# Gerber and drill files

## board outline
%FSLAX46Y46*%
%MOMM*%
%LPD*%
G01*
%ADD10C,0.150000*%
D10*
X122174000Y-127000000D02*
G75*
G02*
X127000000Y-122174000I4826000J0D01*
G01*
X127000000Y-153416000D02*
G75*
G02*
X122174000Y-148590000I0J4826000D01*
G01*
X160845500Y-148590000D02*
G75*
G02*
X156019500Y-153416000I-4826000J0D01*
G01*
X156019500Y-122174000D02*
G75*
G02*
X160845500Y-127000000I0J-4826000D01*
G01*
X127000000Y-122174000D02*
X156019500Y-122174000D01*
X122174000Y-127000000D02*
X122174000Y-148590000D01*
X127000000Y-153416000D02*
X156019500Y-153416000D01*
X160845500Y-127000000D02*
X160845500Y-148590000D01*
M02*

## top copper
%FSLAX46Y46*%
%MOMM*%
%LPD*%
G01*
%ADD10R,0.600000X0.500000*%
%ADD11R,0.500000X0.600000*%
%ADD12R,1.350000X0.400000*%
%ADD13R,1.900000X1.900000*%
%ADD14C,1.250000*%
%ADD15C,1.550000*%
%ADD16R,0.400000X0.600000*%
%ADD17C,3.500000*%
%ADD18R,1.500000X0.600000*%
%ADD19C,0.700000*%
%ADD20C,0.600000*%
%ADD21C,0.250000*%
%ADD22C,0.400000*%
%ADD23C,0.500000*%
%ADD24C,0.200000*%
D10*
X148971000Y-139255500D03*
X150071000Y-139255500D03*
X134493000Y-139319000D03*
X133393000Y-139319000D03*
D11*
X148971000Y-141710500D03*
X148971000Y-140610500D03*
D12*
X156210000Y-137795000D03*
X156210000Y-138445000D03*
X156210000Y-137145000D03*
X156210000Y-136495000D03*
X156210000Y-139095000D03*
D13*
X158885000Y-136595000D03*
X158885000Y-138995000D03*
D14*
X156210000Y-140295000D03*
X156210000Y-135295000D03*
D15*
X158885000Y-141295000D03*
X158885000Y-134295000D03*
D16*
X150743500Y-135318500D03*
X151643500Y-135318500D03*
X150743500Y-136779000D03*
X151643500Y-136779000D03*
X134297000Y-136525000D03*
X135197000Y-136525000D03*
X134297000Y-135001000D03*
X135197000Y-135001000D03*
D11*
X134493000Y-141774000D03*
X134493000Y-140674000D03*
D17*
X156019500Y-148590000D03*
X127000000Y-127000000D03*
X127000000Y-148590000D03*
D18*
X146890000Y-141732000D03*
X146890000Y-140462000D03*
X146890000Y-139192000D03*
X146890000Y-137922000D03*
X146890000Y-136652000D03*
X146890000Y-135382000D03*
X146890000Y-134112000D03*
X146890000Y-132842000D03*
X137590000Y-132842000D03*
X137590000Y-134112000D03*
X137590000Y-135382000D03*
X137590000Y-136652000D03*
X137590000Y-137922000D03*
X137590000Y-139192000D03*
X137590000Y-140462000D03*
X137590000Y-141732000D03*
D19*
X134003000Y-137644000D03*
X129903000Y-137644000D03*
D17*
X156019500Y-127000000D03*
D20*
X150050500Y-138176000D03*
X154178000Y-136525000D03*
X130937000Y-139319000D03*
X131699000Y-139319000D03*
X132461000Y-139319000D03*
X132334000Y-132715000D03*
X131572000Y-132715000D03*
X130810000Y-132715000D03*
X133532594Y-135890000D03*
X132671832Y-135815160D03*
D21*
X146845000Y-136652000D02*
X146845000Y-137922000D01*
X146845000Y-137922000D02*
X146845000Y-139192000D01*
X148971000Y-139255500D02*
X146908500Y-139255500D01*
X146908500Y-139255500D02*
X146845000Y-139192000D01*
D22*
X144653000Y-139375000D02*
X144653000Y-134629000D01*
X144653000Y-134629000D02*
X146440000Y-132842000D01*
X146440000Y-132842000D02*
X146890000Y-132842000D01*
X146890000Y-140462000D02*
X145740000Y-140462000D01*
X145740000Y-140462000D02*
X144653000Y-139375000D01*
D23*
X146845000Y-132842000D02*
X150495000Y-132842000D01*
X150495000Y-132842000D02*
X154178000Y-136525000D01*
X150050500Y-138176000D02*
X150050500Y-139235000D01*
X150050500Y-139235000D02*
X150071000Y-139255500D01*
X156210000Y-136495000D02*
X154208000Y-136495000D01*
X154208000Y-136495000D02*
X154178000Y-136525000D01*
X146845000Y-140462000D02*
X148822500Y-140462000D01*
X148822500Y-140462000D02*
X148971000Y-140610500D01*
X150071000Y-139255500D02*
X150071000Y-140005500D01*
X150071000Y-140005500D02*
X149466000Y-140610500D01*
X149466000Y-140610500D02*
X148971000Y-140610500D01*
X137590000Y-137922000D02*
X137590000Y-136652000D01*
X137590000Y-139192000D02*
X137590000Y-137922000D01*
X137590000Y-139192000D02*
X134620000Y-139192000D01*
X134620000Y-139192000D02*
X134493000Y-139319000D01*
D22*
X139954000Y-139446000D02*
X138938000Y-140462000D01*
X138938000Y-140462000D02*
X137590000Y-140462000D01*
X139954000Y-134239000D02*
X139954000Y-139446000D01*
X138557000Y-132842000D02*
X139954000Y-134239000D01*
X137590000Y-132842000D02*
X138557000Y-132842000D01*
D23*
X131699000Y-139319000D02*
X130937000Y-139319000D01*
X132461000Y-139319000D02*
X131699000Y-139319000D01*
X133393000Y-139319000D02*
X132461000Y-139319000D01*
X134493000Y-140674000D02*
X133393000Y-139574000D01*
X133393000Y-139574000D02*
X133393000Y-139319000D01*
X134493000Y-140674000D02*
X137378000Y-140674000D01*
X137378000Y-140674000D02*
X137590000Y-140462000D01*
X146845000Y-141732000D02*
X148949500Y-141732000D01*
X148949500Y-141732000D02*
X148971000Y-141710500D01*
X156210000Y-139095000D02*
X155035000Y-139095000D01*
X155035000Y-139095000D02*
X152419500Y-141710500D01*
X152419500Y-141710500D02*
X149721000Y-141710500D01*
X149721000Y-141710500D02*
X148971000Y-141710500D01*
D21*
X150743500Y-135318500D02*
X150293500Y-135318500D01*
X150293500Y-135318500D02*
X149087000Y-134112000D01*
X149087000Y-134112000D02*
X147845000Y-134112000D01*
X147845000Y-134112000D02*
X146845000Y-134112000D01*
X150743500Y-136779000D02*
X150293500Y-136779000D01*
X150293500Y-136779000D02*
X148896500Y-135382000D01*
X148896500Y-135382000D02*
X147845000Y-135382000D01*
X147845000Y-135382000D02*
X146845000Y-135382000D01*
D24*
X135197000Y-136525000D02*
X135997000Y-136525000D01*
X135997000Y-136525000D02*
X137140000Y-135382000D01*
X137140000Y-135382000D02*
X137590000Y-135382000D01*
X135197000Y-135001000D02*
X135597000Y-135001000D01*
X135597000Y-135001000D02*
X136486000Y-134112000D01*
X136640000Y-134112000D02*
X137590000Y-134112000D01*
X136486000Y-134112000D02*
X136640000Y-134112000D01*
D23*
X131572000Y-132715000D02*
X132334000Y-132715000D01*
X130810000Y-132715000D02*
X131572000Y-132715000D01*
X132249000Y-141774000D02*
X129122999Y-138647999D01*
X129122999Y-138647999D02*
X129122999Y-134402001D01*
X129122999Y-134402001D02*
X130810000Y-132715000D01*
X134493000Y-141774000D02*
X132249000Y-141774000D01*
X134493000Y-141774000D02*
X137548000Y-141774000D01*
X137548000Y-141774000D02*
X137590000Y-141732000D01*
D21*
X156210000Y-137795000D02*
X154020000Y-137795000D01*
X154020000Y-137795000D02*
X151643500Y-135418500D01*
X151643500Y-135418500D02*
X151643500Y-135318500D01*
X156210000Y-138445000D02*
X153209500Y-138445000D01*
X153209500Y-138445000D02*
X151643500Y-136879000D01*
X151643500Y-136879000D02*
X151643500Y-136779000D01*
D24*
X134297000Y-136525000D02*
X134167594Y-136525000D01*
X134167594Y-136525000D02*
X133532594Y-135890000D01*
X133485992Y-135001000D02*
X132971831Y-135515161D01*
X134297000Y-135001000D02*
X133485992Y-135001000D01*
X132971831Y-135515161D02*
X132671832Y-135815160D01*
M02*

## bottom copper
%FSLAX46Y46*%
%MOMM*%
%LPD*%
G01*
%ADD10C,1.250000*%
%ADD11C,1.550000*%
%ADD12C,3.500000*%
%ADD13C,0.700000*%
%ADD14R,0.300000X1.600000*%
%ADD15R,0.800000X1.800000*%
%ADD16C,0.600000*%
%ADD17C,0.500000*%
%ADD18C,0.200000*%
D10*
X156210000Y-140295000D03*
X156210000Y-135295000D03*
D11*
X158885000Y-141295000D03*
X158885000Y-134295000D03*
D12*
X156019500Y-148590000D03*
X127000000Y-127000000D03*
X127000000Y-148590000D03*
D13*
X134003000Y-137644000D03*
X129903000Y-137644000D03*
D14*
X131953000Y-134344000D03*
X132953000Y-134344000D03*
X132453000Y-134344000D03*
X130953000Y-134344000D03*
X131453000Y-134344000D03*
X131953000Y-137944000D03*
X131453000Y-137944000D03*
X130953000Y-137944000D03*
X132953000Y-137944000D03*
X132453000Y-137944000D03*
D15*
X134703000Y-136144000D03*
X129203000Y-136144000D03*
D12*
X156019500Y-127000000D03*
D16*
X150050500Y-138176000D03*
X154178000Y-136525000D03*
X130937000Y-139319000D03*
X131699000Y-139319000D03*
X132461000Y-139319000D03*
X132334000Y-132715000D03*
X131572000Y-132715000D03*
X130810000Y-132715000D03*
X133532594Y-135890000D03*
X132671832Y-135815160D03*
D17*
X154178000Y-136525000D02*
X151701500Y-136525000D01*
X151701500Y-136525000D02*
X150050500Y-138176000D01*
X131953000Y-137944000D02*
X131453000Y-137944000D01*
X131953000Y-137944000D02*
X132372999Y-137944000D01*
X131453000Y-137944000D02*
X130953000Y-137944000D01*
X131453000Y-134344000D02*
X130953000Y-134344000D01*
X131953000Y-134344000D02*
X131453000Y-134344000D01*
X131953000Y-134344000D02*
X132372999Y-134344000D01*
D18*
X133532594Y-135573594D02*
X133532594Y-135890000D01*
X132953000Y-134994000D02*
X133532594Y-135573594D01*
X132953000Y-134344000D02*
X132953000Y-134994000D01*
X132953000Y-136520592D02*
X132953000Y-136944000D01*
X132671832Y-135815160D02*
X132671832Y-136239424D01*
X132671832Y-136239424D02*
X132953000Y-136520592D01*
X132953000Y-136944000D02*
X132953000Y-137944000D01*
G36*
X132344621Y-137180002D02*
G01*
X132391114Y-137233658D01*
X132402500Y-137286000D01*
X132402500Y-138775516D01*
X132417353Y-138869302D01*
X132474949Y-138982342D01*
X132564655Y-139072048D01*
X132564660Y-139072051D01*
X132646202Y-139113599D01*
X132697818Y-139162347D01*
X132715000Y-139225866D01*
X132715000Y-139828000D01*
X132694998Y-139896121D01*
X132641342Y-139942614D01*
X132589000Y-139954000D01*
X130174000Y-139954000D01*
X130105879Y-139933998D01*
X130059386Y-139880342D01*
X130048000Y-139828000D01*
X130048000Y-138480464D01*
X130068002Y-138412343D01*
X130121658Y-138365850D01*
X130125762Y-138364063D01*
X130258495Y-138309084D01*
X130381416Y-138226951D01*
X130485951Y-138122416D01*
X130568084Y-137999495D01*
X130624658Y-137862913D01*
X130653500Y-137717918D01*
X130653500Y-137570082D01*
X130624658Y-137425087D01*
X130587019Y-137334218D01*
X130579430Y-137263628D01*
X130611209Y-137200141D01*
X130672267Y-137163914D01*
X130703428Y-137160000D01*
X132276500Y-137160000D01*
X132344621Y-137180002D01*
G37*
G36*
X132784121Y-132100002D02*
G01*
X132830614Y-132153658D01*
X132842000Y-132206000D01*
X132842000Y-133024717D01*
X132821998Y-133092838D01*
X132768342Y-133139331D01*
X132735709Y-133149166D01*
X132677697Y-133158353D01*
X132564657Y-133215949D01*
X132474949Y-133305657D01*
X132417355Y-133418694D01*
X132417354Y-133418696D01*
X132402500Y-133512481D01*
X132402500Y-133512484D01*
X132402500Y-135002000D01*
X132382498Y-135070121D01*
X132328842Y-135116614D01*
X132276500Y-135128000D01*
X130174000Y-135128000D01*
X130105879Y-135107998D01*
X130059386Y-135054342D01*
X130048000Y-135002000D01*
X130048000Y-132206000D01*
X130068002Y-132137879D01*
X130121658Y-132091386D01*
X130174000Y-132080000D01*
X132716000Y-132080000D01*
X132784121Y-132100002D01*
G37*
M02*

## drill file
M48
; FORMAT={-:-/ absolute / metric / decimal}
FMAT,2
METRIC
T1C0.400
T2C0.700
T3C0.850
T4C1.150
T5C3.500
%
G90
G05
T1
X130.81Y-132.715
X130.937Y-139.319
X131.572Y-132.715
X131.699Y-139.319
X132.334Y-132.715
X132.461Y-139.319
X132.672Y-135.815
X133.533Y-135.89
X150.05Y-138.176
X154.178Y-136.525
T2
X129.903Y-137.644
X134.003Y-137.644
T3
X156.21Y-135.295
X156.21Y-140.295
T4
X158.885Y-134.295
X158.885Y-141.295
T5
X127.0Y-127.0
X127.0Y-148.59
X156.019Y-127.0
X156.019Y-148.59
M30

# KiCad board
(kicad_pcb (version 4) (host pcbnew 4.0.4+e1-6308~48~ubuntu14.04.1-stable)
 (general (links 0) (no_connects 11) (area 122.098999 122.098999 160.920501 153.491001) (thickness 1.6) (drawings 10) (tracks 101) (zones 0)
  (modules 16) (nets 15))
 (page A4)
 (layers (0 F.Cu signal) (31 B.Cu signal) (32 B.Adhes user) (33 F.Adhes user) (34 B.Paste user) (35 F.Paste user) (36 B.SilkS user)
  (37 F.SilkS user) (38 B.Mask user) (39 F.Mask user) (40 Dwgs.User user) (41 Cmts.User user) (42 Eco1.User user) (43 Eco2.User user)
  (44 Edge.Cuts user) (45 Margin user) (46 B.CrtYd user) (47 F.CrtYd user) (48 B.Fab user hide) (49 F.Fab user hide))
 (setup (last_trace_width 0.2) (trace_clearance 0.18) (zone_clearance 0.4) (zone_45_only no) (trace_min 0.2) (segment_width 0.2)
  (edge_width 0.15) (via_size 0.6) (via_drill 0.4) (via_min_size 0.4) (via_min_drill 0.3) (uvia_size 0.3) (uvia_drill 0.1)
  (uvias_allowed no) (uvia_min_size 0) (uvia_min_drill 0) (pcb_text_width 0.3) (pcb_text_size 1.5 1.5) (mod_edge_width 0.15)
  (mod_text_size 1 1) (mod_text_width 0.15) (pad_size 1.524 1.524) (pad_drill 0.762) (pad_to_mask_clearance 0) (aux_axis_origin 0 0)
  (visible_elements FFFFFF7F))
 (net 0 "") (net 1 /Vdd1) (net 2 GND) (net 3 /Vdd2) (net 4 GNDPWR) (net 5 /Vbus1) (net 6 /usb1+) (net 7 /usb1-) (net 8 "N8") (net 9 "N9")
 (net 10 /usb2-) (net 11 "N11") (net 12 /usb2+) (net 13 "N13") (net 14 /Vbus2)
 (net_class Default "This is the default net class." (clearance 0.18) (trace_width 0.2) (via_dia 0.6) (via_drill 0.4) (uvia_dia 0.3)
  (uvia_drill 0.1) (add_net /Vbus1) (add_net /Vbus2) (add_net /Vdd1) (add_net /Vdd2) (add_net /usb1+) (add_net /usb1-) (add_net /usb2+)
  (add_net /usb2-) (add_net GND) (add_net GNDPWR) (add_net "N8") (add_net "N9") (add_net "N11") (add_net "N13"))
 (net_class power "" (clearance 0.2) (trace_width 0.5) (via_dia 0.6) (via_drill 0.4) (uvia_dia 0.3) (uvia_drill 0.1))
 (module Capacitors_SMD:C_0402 (layer F.Cu) (at 149.521 139.2555)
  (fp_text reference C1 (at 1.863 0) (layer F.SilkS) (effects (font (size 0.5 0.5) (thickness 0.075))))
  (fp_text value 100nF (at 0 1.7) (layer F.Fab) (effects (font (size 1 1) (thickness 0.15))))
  (pad 1 smd rect (at -0.55 0) (size 0.6 0.5) (layers F.Cu F.Paste F.Mask) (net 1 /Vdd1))
  (pad 2 smd rect (at 0.55 0) (size 0.6 0.5) (layers F.Cu F.Paste F.Mask) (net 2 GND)))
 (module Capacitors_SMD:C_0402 (layer F.Cu) (at 133.943 139.319 180)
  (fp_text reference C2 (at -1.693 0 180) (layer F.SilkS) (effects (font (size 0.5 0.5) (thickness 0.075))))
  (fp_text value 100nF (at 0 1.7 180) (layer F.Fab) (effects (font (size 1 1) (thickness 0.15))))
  (pad 1 smd rect (at -0.55 0 180) (size 0.6 0.5) (layers F.Cu F.Paste F.Mask) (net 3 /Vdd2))
  (pad 2 smd rect (at 0.55 0 180) (size 0.6 0.5) (layers F.Cu F.Paste F.Mask) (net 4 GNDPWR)))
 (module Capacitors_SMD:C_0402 (layer F.Cu) (at 148.971 141.1605 90)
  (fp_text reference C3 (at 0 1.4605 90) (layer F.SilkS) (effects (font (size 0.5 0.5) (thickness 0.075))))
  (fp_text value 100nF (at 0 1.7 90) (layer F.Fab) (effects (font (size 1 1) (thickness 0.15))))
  (pad 1 smd rect (at -0.55 0 90) (size 0.6 0.5) (layers F.Cu F.Paste F.Mask) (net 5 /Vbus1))
  (pad 2 smd rect (at 0.55 0 90) (size 0.6 0.5) (layers F.Cu F.Paste F.Mask) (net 2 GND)))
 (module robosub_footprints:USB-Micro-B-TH (layer F.Cu) (at 155.535 137.795 90)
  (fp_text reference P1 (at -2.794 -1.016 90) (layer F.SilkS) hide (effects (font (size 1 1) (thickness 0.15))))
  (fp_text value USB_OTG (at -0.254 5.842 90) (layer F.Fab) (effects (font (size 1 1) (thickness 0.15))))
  (pad 3 smd rect (at 0 0.675 90) (size 0.4 1.35) (layers F.Cu F.Paste F.Mask) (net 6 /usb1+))
  (pad 2 smd rect (at -0.65 0.675 90) (size 0.4 1.35) (layers F.Cu F.Paste F.Mask) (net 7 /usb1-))
  (pad 4 smd rect (at 0.65 0.675 90) (size 0.4 1.35) (layers F.Cu F.Paste F.Mask))
  (pad 5 smd rect (at 1.3 0.675 90) (size 0.4 1.35) (layers F.Cu F.Paste F.Mask) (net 2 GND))
  (pad 1 smd rect (at -1.3 0.675 90) (size 0.4 1.35) (layers F.Cu F.Paste F.Mask) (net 5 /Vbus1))
  (pad "" smd rect (at 1.2 3.35 90) (size 1.9 1.9) (layers F.Cu F.Paste F.Mask))
  (pad "" smd rect (at -1.2 3.35 90) (size 1.9 1.9) (layers F.Cu F.Paste F.Mask))
  (pad "" thru_hole circle (at -2.5 0.675 90) (size 1.25 1.25) (drill 0.85) (layers *.Cu *.Mask F.SilkS))
  (pad "" thru_hole circle (at 2.5 0.675 90) (size 1.25 1.25) (drill 0.85) (layers *.Cu *.Mask F.SilkS))
  (pad "" thru_hole circle (at -3.5 3.35 90) (size 1.55 1.55) (drill 1.15) (layers *.Cu *.Mask F.SilkS))
  (pad "" thru_hole circle (at 3.5 3.35 90) (size 1.55 1.55) (drill 1.15) (layers *.Cu *.Mask F.SilkS)))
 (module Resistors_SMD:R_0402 (layer F.Cu) (at 151.1935 135.3185)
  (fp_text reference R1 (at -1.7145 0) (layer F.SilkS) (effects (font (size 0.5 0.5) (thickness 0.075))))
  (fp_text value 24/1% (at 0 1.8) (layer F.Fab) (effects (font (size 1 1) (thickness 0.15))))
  (pad 1 smd rect (at -0.45 0) (size 0.4 0.6) (layers F.Cu F.Paste F.Mask) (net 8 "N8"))
  (pad 2 smd rect (at 0.45 0) (size 0.4 0.6) (layers F.Cu F.Paste F.Mask) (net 6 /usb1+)))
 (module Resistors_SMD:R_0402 (layer F.Cu) (at 151.1935 136.779)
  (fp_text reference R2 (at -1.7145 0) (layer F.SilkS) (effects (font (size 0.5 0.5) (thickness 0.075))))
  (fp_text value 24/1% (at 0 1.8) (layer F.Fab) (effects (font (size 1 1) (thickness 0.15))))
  (pad 1 smd rect (at -0.45 0) (size 0.4 0.6) (layers F.Cu F.Paste F.Mask) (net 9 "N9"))
  (pad 2 smd rect (at 0.45 0) (size 0.4 0.6) (layers F.Cu F.Paste F.Mask) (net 7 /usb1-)))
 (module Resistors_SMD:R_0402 (layer F.Cu) (at 134.747 136.525)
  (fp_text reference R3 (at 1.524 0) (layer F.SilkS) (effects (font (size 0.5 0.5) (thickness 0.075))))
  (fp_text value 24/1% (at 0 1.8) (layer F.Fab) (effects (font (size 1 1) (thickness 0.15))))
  (pad 1 smd rect (at -0.45 0) (size 0.4 0.6) (layers F.Cu F.Paste F.Mask) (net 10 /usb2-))
  (pad 2 smd rect (at 0.45 0) (size 0.4 0.6) (layers F.Cu F.Paste F.Mask) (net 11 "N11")))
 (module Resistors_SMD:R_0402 (layer F.Cu) (at 134.747 135.001)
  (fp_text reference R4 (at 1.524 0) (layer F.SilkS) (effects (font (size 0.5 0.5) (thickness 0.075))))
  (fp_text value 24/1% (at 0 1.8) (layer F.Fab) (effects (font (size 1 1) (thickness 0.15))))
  (pad 1 smd rect (at -0.45 0) (size 0.4 0.6) (layers F.Cu F.Paste F.Mask) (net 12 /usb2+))
  (pad 2 smd rect (at 0.45 0) (size 0.4 0.6) (layers F.Cu F.Paste F.Mask) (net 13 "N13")))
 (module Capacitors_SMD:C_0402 (layer F.Cu) (at 134.493 141.224 90)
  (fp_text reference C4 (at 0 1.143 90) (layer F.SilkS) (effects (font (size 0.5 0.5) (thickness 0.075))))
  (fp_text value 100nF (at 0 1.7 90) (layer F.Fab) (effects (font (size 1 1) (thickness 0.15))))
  (pad 1 smd rect (at -0.55 0 90) (size 0.6 0.5) (layers F.Cu F.Paste F.Mask) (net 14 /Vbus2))
  (pad 2 smd rect (at 0.55 0 90) (size 0.6 0.5) (layers F.Cu F.Paste F.Mask) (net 4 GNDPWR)))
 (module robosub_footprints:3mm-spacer (layer F.Cu) (at 156.0195 148.59)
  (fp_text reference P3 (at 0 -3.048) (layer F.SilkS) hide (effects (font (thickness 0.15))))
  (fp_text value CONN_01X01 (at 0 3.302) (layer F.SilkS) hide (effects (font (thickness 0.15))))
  (pad "" thru_hole circle (at 0 0) (size 3.5 3.5) (drill 3.5) (layers *.Cu *.Mask F.SilkS)))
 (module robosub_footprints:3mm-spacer (layer F.Cu) (at 127 127)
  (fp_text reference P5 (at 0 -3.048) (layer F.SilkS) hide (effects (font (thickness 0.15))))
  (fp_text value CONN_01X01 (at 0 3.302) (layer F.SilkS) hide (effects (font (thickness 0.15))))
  (pad "" thru_hole circle (at 0 0) (size 3.5 3.5) (drill 3.5) (layers *.Cu *.Mask F.SilkS)))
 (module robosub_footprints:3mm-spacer (layer F.Cu) (at 127 148.59)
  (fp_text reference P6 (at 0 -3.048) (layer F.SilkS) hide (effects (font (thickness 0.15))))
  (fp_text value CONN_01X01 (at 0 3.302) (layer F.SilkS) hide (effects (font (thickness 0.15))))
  (pad "" thru_hole circle (at 0 0) (size 3.5 3.5) (drill 3.5) (layers *.Cu *.Mask F.SilkS)))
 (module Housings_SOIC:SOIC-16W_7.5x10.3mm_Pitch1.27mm (layer F.Cu) (at 142.24 137.287 180)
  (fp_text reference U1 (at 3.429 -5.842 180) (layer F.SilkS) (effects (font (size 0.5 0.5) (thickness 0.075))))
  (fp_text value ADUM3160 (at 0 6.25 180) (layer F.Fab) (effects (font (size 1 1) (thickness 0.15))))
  (pad 1 smd rect (at -4.65 -4.445 180) (size 1.5 0.6) (layers F.Cu F.Paste F.Mask) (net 5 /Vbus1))
  (pad 2 smd rect (at -4.65 -3.175 180) (size 1.5 0.6) (layers F.Cu F.Paste F.Mask) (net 2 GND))
  (pad 3 smd rect (at -4.65 -1.905 180) (size 1.5 0.6) (layers F.Cu F.Paste F.Mask) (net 1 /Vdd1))
  (pad 4 smd rect (at -4.65 -0.635 180) (size 1.5 0.6) (layers F.Cu F.Paste F.Mask) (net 1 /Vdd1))
  (pad 5 smd rect (at -4.65 0.635 180) (size 1.5 0.6) (layers F.Cu F.Paste F.Mask) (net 1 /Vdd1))
  (pad 6 smd rect (at -4.65 1.905 180) (size 1.5 0.6) (layers F.Cu F.Paste F.Mask) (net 9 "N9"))
  (pad 7 smd rect (at -4.65 3.175 180) (size 1.5 0.6) (layers F.Cu F.Paste F.Mask) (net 8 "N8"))
  (pad 8 smd rect (at -4.65 4.445 180) (size 1.5 0.6) (layers F.Cu F.Paste F.Mask) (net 2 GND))
  (pad 9 smd rect (at 4.65 4.445 180) (size 1.5 0.6) (layers F.Cu F.Paste F.Mask) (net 4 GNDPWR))
  (pad 10 smd rect (at 4.65 3.175 180) (size 1.5 0.6) (layers F.Cu F.Paste F.Mask) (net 13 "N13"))
  (pad 11 smd rect (at 4.65 1.905 180) (size 1.5 0.6) (layers F.Cu F.Paste F.Mask) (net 11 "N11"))
  (pad 12 smd rect (at 4.65 0.635 180) (size 1.5 0.6) (layers F.Cu F.Paste F.Mask) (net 3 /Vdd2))
  (pad 13 smd rect (at 4.65 -0.635 180) (size 1.5 0.6) (layers F.Cu F.Paste F.Mask) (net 3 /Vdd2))
  (pad 14 smd rect (at 4.65 -1.905 180) (size 1.5 0.6) (layers F.Cu F.Paste F.Mask) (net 3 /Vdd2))
  (pad 15 smd rect (at 4.65 -3.175 180) (size 1.5 0.6) (layers F.Cu F.Paste F.Mask) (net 4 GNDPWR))
  (pad 16 smd rect (at 4.65 -4.445 180) (size 1.5 0.6) (layers F.Cu F.Paste F.Mask) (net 14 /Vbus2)))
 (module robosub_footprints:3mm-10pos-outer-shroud (layer B.Cu) (at 131.953 136.144)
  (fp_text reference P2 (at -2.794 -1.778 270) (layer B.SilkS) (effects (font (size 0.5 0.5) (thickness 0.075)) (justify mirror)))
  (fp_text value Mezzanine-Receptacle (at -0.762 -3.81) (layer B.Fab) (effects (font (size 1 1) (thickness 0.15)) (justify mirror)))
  (pad "" thru_hole circle (at 2.05 1.5) (size 0.7 0.7) (drill 0.7) (layers *.Cu *.Mask))
  (pad "" thru_hole circle (at -2.05 1.5) (size 0.7 0.7) (drill 0.7) (layers *.Cu *.Mask))
  (pad 5 smd rect (at 0 -1.8) (size 0.3 1.6) (layers B.Cu B.Paste B.Mask) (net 14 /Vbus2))
  (pad 9 smd rect (at 1 -1.8) (size 0.3 1.6) (layers B.Cu B.Paste B.Mask) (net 10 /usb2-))
  (pad 7 smd rect (at 0.5 -1.8) (size 0.3 1.6) (layers B.Cu B.Paste B.Mask) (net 14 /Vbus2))
  (pad 1 smd rect (at -1 -1.8) (size 0.3 1.6) (layers B.Cu B.Paste B.Mask) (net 14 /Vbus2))
  (pad 3 smd rect (at -0.5 -1.8) (size 0.3 1.6) (layers B.Cu B.Paste B.Mask) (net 14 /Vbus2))
  (pad 6 smd rect (at 0 1.8) (size 0.3 1.6) (layers B.Cu B.Paste B.Mask) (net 4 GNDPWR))
  (pad 4 smd rect (at -0.5 1.8) (size 0.3 1.6) (layers B.Cu B.Paste B.Mask) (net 4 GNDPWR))
  (pad 2 smd rect (at -1 1.8) (size 0.3 1.6) (layers B.Cu B.Paste B.Mask) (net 4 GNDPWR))
  (pad 10 smd rect (at 1 1.8) (size 0.3 1.6) (layers B.Cu B.Paste B.Mask) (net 12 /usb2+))
  (pad 8 smd rect (at 0.5 1.8) (size 0.3 1.6) (layers B.Cu B.Paste B.Mask) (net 4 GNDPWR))
  (pad "" smd rect (at 2.75 0) (size 0.8 1.8) (layers B.Cu B.Paste B.Mask))
  (pad "" smd rect (at -2.75 0) (size 0.8 1.8) (layers B.Cu B.Paste B.Mask)))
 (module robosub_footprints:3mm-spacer (layer F.Cu) (at 156.0195 127)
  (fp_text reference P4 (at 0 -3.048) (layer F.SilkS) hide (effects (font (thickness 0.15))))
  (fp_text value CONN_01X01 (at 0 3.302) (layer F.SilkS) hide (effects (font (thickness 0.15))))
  (pad "" thru_hole circle (at 0 0) (size 3.5 3.5) (drill 3.5) (layers *.Cu *.Mask F.SilkS)))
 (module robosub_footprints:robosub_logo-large (layer F.Cu) (at 141.732 148.717)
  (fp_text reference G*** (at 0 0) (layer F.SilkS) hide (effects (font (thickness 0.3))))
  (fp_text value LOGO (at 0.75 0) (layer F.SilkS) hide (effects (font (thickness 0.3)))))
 (gr_arc (start 127 127) (end 122.174 127) (angle 90) (layer Edge.Cuts) (width 0.15))
 (gr_arc (start 127 148.59) (end 127 153.416) (angle 90) (layer Edge.Cuts) (width 0.15))
 (gr_arc (start 156.0195 148.59) (end 160.8455 148.59) (angle 90) (layer Edge.Cuts) (width 0.15))
 (gr_arc (start 156.0195 127) (end 156.0195 122.174) (angle 90) (layer Edge.Cuts) (width 0.15))
 (gr_line (start 127 122.174) (end 156.0195 122.174) (layer Edge.Cuts) (width 0.15))
 (gr_line (start 122.174 127) (end 122.174 148.59) (layer Edge.Cuts) (width 0.15))
 (gr_line (start 127 153.416) (end 156.0195 153.416) (layer Edge.Cuts) (width 0.15))
 (gr_line (start 160.8455 127) (end 160.8455 148.59) (layer Edge.Cuts) (width 0.15))
 (segment (start 146.845 136.652) (end 146.845 137.922) (width 0.25) (layer F.Cu) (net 1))
 (segment (start 146.845 137.922) (end 146.845 139.192) (width 0.25) (layer F.Cu) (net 1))
 (segment (start 148.971 139.2555) (end 146.9085 139.2555) (width 0.25) (layer F.Cu) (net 1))
 (segment (start 146.9085 139.2555) (end 146.845 139.192) (width 0.25) (layer F.Cu) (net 1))
 (segment (start 144.653 139.375) (end 144.653 134.629) (width 0.4) (layer F.Cu) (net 2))
 (segment (start 144.653 134.629) (end 146.44 132.842) (width 0.4) (layer F.Cu) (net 2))
 (segment (start 146.44 132.842) (end 146.89 132.842) (width 0.4) (layer F.Cu) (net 2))
 (segment (start 146.89 140.462) (end 145.74 140.462) (width 0.4) (layer F.Cu) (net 2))
 (segment (start 145.74 140.462) (end 144.653 139.375) (width 0.4) (layer F.Cu) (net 2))
 (segment (start 146.845 132.842) (end 150.495 132.842) (width 0.5) (layer F.Cu) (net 2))
 (segment (start 150.495 132.842) (end 154.178 136.525) (width 0.5) (layer F.Cu) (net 2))
 (segment (start 150.0505 138.176) (end 150.0505 139.235) (width 0.5) (layer F.Cu) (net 2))
 (segment (start 150.0505 139.235) (end 150.071 139.2555) (width 0.5) (layer F.Cu) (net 2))
 (segment (start 154.178 136.525) (end 151.7015 136.525) (width 0.5) (layer B.Cu) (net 2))
 (segment (start 151.7015 136.525) (end 150.0505 138.176) (width 0.5) (layer B.Cu) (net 2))
 (via (at 150.0505 138.176) (size 0.6) (drill 0.4) (layers F.Cu B.Cu) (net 2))
 (segment (start 156.21 136.495) (end 154.208 136.495) (width 0.5) (layer F.Cu) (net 2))
 (segment (start 154.208 136.495) (end 154.178 136.525) (width 0.5) (layer F.Cu) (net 2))
 (via (at 154.178 136.525) (size 0.6) (drill 0.4) (layers F.Cu B.Cu) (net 2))
 (segment (start 146.845 140.462) (end 148.8225 140.462) (width 0.5) (layer F.Cu) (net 2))
 (segment (start 148.8225 140.462) (end 148.971 140.6105) (width 0.5) (layer F.Cu) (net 2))
 (segment (start 150.071 139.2555) (end 150.071 140.0055) (width 0.5) (layer F.Cu) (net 2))
 (segment (start 150.071 140.0055) (end 149.466 140.6105) (width 0.5) (layer F.Cu) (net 2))
 (segment (start 149.466 140.6105) (end 148.971 140.6105) (width 0.5) (layer F.Cu) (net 2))
 (segment (start 137.59 137.922) (end 137.59 136.652) (width 0.5) (layer F.Cu) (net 3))
 (segment (start 137.59 139.192) (end 137.59 137.922) (width 0.5) (layer F.Cu) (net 3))
 (segment (start 137.59 139.192) (end 134.62 139.192) (width 0.5) (layer F.Cu) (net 3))
 (segment (start 134.62 139.192) (end 134.493 139.319) (width 0.5) (layer F.Cu) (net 3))
 (segment (start 139.954 139.446) (end 138.938 140.462) (width 0.4) (layer F.Cu) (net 4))
 (segment (start 138.938 140.462) (end 137.59 140.462) (width 0.4) (layer F.Cu) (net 4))
 (segment (start 139.954 134.239) (end 139.954 139.446) (width 0.4) (layer F.Cu) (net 4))
 (segment (start 138.557 132.842) (end 139.954 134.239) (width 0.4) (layer F.Cu) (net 4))
 (segment (start 137.59 132.842) (end 138.557 132.842) (width 0.4) (layer F.Cu) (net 4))
 (segment (start 131.953 137.944) (end 131.453 137.944) (width 0.5) (layer B.Cu) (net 4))
 (segment (start 131.699 139.319) (end 130.937 139.319) (width 0.5) (layer F.Cu) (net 4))
 (via (at 130.937 139.319) (size 0.6) (drill 0.4) (layers F.Cu B.Cu) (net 4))
 (segment (start 132.461 139.319) (end 131.699 139.319) (width 0.5) (layer F.Cu) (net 4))
 (via (at 131.699 139.319) (size 0.6) (drill 0.4) (layers F.Cu B.Cu) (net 4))
 (segment (start 133.393 139.319) (end 132.461 139.319) (width 0.5) (layer F.Cu) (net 4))
 (via (at 132.461 139.319) (size 0.6) (drill 0.4) (layers F.Cu B.Cu) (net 4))
 (segment (start 131.953 137.944) (end 132.372999 137.944) (width 0.5) (layer B.Cu) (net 4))
 (segment (start 131.453 137.944) (end 130.953 137.944) (width 0.5) (layer B.Cu) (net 4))
 (segment (start 134.493 140.674) (end 133.393 139.574) (width 0.5) (layer F.Cu) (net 4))
 (segment (start 133.393 139.574) (end 133.393 139.319) (width 0.5) (layer F.Cu) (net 4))
 (segment (start 134.493 140.674) (end 137.378 140.674) (width 0.5) (layer F.Cu) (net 4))
 (segment (start 137.378 140.674) (end 137.59 140.462) (width 0.5) (layer F.Cu) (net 4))
 (segment (start 146.845 141.732) (end 148.9495 141.732) (width 0.5) (layer F.Cu) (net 5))
 (segment (start 148.9495 141.732) (end 148.971 141.7105) (width 0.5) (layer F.Cu) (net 5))
 (segment (start 156.21 139.095) (end 155.035 139.095) (width 0.5) (layer F.Cu) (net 5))
 (segment (start 155.035 139.095) (end 152.4195 141.7105) (width 0.5) (layer F.Cu) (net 5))
 (segment (start 152.4195 141.7105) (end 149.721 141.7105) (width 0.5) (layer F.Cu) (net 5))
 (segment (start 149.721 141.7105) (end 148.971 141.7105) (width 0.5) (layer F.Cu) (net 5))
 (segment (start 150.7435 135.3185) (end 150.2935 135.3185) (width 0.25) (layer F.Cu) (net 8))
 (segment (start 150.2935 135.3185) (end 149.087 134.112) (width 0.25) (layer F.Cu) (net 8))
 (segment (start 149.087 134.112) (end 147.845 134.112) (width 0.25) (layer F.Cu) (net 8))
 (segment (start 147.845 134.112) (end 146.845 134.112) (width 0.25) (layer F.Cu) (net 8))
 (segment (start 150.7435 136.779) (end 150.2935 136.779) (width 0.25) (layer F.Cu) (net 9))
 (segment (start 150.2935 136.779) (end 148.8965 135.382) (width 0.25) (layer F.Cu) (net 9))
 (segment (start 148.8965 135.382) (end 147.845 135.382) (width 0.25) (layer F.Cu) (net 9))
 (segment (start 147.845 135.382) (end 146.845 135.382) (width 0.25) (layer F.Cu) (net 9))
 (segment (start 135.197 136.525) (end 135.997 136.525) (width 0.2) (layer F.Cu) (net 11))
 (segment (start 135.997 136.525) (end 137.14 135.382) (width 0.2) (layer F.Cu) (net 11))
 (segment (start 137.14 135.382) (end 137.59 135.382) (width 0.2) (layer F.Cu) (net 11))
 (segment (start 135.197 135.001) (end 135.597 135.001) (width 0.2) (layer F.Cu) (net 13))
 (segment (start 135.597 135.001) (end 136.486 134.112) (width 0.2) (layer F.Cu) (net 13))
 (segment (start 136.64 134.112) (end 137.59 134.112) (width 0.2) (layer F.Cu) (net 13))
 (segment (start 136.486 134.112) (end 136.64 134.112) (width 0.2) (layer F.Cu) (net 13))
 (segment (start 131.453 134.344) (end 130.953 134.344) (width 0.5) (layer B.Cu) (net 14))
 (segment (start 131.953 134.344) (end 131.453 134.344) (width 0.5) (layer B.Cu) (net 14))
 (segment (start 131.953 134.344) (end 132.372999 134.344) (width 0.5) (layer B.Cu) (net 14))
 (segment (start 131.572 132.715) (end 132.334 132.715) (width 0.5) (layer F.Cu) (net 14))
 (via (at 132.334 132.715) (size 0.6) (drill 0.4) (layers F.Cu B.Cu) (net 14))
 (segment (start 130.81 132.715) (end 131.572 132.715) (width 0.5) (layer F.Cu) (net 14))
 (via (at 131.572 132.715) (size 0.6) (drill 0.4) (layers F.Cu B.Cu) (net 14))
 (segment (start 132.249 141.774) (end 129.122999 138.647999) (width 0.5) (layer F.Cu) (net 14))
 (segment (start 129.122999 138.647999) (end 129.122999 134.402001) (width 0.5) (layer F.Cu) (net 14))
 (segment (start 129.122999 134.402001) (end 130.81 132.715) (width 0.5) (layer F.Cu) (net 14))
 (via (at 130.81 132.715) (size 0.6) (drill 0.4) (layers F.Cu B.Cu) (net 14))
 (segment (start 134.493 141.774) (end 132.249 141.774) (width 0.5) (layer F.Cu) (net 14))
 (segment (start 134.493 141.774) (end 137.548 141.774) (width 0.5) (layer F.Cu) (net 14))
 (segment (start 137.548 141.774) (end 137.59 141.732) (width 0.5) (layer F.Cu) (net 14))
 (segment (start 156.21 137.795) (end 154.02 137.795) (width 0.25) (layer F.Cu) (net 6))
 (segment (start 154.02 137.795) (end 151.6435 135.4185) (width 0.25) (layer F.Cu) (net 6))
 (segment (start 151.6435 135.4185) (end 151.6435 135.3185) (width 0.25) (layer F.Cu) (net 6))
 (segment (start 156.21 138.445) (end 153.2095 138.445) (width 0.25) (layer F.Cu) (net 7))
 (segment (start 153.2095 138.445) (end 151.6435 136.879) (width 0.25) (layer F.Cu) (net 7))
 (segment (start 151.6435 136.879) (end 151.6435 136.779) (width 0.25) (layer F.Cu) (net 7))
 (segment (start 133.532594 135.573594) (end 133.532594 135.89) (width 0.2) (layer B.Cu) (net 10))
 (segment (start 134.297 136.525) (end 134.167594 136.525) (width 0.2) (layer F.Cu) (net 10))
 (segment (start 134.167594 136.525) (end 133.532594 135.89) (width 0.2) (layer F.Cu) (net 10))
 (via (at 133.532594 135.89) (size 0.6) (drill 0.4) (layers F.Cu B.Cu) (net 10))
 (segment (start 132.953 134.994) (end 133.532594 135.573594) (width 0.2) (layer B.Cu) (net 10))
 (segment (start 132.953 134.344) (end 132.953 134.994) (width 0.2) (layer B.Cu) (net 10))
 (segment (start 132.953 136.520592) (end 132.953 136.944) (width 0.2) (layer B.Cu) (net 12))
 (segment (start 132.671832 135.81516) (end 132.671832 136.239424) (width 0.2) (layer B.Cu) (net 12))
 (segment (start 132.671832 136.239424) (end 132.953 136.520592) (width 0.2) (layer B.Cu) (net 12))
 (segment (start 132.953 136.944) (end 132.953 137.944) (width 0.2) (layer B.Cu) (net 12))
 (segment (start 133.485992 135.001) (end 132.971831 135.515161) (width 0.2) (layer F.Cu) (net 12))
 (segment (start 134.297 135.001) (end 133.485992 135.001) (width 0.2) (layer F.Cu) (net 12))
 (via (at 132.671832 135.81516) (size 0.6) (drill 0.4) (layers F.Cu B.Cu) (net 12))
 (segment (start 132.971831 135.515161) (end 132.671832 135.81516) (width 0.2) (layer F.Cu) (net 12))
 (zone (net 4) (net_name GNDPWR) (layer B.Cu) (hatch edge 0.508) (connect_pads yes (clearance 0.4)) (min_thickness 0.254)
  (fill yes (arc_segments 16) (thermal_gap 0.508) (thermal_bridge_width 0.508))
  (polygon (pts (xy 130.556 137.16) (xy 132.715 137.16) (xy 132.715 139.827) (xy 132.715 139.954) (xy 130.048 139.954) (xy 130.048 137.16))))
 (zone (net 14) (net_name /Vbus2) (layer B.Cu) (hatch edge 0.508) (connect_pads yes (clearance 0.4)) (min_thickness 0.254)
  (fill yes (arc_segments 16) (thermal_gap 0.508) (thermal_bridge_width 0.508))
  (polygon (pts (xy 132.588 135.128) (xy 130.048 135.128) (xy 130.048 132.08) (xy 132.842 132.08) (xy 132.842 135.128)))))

